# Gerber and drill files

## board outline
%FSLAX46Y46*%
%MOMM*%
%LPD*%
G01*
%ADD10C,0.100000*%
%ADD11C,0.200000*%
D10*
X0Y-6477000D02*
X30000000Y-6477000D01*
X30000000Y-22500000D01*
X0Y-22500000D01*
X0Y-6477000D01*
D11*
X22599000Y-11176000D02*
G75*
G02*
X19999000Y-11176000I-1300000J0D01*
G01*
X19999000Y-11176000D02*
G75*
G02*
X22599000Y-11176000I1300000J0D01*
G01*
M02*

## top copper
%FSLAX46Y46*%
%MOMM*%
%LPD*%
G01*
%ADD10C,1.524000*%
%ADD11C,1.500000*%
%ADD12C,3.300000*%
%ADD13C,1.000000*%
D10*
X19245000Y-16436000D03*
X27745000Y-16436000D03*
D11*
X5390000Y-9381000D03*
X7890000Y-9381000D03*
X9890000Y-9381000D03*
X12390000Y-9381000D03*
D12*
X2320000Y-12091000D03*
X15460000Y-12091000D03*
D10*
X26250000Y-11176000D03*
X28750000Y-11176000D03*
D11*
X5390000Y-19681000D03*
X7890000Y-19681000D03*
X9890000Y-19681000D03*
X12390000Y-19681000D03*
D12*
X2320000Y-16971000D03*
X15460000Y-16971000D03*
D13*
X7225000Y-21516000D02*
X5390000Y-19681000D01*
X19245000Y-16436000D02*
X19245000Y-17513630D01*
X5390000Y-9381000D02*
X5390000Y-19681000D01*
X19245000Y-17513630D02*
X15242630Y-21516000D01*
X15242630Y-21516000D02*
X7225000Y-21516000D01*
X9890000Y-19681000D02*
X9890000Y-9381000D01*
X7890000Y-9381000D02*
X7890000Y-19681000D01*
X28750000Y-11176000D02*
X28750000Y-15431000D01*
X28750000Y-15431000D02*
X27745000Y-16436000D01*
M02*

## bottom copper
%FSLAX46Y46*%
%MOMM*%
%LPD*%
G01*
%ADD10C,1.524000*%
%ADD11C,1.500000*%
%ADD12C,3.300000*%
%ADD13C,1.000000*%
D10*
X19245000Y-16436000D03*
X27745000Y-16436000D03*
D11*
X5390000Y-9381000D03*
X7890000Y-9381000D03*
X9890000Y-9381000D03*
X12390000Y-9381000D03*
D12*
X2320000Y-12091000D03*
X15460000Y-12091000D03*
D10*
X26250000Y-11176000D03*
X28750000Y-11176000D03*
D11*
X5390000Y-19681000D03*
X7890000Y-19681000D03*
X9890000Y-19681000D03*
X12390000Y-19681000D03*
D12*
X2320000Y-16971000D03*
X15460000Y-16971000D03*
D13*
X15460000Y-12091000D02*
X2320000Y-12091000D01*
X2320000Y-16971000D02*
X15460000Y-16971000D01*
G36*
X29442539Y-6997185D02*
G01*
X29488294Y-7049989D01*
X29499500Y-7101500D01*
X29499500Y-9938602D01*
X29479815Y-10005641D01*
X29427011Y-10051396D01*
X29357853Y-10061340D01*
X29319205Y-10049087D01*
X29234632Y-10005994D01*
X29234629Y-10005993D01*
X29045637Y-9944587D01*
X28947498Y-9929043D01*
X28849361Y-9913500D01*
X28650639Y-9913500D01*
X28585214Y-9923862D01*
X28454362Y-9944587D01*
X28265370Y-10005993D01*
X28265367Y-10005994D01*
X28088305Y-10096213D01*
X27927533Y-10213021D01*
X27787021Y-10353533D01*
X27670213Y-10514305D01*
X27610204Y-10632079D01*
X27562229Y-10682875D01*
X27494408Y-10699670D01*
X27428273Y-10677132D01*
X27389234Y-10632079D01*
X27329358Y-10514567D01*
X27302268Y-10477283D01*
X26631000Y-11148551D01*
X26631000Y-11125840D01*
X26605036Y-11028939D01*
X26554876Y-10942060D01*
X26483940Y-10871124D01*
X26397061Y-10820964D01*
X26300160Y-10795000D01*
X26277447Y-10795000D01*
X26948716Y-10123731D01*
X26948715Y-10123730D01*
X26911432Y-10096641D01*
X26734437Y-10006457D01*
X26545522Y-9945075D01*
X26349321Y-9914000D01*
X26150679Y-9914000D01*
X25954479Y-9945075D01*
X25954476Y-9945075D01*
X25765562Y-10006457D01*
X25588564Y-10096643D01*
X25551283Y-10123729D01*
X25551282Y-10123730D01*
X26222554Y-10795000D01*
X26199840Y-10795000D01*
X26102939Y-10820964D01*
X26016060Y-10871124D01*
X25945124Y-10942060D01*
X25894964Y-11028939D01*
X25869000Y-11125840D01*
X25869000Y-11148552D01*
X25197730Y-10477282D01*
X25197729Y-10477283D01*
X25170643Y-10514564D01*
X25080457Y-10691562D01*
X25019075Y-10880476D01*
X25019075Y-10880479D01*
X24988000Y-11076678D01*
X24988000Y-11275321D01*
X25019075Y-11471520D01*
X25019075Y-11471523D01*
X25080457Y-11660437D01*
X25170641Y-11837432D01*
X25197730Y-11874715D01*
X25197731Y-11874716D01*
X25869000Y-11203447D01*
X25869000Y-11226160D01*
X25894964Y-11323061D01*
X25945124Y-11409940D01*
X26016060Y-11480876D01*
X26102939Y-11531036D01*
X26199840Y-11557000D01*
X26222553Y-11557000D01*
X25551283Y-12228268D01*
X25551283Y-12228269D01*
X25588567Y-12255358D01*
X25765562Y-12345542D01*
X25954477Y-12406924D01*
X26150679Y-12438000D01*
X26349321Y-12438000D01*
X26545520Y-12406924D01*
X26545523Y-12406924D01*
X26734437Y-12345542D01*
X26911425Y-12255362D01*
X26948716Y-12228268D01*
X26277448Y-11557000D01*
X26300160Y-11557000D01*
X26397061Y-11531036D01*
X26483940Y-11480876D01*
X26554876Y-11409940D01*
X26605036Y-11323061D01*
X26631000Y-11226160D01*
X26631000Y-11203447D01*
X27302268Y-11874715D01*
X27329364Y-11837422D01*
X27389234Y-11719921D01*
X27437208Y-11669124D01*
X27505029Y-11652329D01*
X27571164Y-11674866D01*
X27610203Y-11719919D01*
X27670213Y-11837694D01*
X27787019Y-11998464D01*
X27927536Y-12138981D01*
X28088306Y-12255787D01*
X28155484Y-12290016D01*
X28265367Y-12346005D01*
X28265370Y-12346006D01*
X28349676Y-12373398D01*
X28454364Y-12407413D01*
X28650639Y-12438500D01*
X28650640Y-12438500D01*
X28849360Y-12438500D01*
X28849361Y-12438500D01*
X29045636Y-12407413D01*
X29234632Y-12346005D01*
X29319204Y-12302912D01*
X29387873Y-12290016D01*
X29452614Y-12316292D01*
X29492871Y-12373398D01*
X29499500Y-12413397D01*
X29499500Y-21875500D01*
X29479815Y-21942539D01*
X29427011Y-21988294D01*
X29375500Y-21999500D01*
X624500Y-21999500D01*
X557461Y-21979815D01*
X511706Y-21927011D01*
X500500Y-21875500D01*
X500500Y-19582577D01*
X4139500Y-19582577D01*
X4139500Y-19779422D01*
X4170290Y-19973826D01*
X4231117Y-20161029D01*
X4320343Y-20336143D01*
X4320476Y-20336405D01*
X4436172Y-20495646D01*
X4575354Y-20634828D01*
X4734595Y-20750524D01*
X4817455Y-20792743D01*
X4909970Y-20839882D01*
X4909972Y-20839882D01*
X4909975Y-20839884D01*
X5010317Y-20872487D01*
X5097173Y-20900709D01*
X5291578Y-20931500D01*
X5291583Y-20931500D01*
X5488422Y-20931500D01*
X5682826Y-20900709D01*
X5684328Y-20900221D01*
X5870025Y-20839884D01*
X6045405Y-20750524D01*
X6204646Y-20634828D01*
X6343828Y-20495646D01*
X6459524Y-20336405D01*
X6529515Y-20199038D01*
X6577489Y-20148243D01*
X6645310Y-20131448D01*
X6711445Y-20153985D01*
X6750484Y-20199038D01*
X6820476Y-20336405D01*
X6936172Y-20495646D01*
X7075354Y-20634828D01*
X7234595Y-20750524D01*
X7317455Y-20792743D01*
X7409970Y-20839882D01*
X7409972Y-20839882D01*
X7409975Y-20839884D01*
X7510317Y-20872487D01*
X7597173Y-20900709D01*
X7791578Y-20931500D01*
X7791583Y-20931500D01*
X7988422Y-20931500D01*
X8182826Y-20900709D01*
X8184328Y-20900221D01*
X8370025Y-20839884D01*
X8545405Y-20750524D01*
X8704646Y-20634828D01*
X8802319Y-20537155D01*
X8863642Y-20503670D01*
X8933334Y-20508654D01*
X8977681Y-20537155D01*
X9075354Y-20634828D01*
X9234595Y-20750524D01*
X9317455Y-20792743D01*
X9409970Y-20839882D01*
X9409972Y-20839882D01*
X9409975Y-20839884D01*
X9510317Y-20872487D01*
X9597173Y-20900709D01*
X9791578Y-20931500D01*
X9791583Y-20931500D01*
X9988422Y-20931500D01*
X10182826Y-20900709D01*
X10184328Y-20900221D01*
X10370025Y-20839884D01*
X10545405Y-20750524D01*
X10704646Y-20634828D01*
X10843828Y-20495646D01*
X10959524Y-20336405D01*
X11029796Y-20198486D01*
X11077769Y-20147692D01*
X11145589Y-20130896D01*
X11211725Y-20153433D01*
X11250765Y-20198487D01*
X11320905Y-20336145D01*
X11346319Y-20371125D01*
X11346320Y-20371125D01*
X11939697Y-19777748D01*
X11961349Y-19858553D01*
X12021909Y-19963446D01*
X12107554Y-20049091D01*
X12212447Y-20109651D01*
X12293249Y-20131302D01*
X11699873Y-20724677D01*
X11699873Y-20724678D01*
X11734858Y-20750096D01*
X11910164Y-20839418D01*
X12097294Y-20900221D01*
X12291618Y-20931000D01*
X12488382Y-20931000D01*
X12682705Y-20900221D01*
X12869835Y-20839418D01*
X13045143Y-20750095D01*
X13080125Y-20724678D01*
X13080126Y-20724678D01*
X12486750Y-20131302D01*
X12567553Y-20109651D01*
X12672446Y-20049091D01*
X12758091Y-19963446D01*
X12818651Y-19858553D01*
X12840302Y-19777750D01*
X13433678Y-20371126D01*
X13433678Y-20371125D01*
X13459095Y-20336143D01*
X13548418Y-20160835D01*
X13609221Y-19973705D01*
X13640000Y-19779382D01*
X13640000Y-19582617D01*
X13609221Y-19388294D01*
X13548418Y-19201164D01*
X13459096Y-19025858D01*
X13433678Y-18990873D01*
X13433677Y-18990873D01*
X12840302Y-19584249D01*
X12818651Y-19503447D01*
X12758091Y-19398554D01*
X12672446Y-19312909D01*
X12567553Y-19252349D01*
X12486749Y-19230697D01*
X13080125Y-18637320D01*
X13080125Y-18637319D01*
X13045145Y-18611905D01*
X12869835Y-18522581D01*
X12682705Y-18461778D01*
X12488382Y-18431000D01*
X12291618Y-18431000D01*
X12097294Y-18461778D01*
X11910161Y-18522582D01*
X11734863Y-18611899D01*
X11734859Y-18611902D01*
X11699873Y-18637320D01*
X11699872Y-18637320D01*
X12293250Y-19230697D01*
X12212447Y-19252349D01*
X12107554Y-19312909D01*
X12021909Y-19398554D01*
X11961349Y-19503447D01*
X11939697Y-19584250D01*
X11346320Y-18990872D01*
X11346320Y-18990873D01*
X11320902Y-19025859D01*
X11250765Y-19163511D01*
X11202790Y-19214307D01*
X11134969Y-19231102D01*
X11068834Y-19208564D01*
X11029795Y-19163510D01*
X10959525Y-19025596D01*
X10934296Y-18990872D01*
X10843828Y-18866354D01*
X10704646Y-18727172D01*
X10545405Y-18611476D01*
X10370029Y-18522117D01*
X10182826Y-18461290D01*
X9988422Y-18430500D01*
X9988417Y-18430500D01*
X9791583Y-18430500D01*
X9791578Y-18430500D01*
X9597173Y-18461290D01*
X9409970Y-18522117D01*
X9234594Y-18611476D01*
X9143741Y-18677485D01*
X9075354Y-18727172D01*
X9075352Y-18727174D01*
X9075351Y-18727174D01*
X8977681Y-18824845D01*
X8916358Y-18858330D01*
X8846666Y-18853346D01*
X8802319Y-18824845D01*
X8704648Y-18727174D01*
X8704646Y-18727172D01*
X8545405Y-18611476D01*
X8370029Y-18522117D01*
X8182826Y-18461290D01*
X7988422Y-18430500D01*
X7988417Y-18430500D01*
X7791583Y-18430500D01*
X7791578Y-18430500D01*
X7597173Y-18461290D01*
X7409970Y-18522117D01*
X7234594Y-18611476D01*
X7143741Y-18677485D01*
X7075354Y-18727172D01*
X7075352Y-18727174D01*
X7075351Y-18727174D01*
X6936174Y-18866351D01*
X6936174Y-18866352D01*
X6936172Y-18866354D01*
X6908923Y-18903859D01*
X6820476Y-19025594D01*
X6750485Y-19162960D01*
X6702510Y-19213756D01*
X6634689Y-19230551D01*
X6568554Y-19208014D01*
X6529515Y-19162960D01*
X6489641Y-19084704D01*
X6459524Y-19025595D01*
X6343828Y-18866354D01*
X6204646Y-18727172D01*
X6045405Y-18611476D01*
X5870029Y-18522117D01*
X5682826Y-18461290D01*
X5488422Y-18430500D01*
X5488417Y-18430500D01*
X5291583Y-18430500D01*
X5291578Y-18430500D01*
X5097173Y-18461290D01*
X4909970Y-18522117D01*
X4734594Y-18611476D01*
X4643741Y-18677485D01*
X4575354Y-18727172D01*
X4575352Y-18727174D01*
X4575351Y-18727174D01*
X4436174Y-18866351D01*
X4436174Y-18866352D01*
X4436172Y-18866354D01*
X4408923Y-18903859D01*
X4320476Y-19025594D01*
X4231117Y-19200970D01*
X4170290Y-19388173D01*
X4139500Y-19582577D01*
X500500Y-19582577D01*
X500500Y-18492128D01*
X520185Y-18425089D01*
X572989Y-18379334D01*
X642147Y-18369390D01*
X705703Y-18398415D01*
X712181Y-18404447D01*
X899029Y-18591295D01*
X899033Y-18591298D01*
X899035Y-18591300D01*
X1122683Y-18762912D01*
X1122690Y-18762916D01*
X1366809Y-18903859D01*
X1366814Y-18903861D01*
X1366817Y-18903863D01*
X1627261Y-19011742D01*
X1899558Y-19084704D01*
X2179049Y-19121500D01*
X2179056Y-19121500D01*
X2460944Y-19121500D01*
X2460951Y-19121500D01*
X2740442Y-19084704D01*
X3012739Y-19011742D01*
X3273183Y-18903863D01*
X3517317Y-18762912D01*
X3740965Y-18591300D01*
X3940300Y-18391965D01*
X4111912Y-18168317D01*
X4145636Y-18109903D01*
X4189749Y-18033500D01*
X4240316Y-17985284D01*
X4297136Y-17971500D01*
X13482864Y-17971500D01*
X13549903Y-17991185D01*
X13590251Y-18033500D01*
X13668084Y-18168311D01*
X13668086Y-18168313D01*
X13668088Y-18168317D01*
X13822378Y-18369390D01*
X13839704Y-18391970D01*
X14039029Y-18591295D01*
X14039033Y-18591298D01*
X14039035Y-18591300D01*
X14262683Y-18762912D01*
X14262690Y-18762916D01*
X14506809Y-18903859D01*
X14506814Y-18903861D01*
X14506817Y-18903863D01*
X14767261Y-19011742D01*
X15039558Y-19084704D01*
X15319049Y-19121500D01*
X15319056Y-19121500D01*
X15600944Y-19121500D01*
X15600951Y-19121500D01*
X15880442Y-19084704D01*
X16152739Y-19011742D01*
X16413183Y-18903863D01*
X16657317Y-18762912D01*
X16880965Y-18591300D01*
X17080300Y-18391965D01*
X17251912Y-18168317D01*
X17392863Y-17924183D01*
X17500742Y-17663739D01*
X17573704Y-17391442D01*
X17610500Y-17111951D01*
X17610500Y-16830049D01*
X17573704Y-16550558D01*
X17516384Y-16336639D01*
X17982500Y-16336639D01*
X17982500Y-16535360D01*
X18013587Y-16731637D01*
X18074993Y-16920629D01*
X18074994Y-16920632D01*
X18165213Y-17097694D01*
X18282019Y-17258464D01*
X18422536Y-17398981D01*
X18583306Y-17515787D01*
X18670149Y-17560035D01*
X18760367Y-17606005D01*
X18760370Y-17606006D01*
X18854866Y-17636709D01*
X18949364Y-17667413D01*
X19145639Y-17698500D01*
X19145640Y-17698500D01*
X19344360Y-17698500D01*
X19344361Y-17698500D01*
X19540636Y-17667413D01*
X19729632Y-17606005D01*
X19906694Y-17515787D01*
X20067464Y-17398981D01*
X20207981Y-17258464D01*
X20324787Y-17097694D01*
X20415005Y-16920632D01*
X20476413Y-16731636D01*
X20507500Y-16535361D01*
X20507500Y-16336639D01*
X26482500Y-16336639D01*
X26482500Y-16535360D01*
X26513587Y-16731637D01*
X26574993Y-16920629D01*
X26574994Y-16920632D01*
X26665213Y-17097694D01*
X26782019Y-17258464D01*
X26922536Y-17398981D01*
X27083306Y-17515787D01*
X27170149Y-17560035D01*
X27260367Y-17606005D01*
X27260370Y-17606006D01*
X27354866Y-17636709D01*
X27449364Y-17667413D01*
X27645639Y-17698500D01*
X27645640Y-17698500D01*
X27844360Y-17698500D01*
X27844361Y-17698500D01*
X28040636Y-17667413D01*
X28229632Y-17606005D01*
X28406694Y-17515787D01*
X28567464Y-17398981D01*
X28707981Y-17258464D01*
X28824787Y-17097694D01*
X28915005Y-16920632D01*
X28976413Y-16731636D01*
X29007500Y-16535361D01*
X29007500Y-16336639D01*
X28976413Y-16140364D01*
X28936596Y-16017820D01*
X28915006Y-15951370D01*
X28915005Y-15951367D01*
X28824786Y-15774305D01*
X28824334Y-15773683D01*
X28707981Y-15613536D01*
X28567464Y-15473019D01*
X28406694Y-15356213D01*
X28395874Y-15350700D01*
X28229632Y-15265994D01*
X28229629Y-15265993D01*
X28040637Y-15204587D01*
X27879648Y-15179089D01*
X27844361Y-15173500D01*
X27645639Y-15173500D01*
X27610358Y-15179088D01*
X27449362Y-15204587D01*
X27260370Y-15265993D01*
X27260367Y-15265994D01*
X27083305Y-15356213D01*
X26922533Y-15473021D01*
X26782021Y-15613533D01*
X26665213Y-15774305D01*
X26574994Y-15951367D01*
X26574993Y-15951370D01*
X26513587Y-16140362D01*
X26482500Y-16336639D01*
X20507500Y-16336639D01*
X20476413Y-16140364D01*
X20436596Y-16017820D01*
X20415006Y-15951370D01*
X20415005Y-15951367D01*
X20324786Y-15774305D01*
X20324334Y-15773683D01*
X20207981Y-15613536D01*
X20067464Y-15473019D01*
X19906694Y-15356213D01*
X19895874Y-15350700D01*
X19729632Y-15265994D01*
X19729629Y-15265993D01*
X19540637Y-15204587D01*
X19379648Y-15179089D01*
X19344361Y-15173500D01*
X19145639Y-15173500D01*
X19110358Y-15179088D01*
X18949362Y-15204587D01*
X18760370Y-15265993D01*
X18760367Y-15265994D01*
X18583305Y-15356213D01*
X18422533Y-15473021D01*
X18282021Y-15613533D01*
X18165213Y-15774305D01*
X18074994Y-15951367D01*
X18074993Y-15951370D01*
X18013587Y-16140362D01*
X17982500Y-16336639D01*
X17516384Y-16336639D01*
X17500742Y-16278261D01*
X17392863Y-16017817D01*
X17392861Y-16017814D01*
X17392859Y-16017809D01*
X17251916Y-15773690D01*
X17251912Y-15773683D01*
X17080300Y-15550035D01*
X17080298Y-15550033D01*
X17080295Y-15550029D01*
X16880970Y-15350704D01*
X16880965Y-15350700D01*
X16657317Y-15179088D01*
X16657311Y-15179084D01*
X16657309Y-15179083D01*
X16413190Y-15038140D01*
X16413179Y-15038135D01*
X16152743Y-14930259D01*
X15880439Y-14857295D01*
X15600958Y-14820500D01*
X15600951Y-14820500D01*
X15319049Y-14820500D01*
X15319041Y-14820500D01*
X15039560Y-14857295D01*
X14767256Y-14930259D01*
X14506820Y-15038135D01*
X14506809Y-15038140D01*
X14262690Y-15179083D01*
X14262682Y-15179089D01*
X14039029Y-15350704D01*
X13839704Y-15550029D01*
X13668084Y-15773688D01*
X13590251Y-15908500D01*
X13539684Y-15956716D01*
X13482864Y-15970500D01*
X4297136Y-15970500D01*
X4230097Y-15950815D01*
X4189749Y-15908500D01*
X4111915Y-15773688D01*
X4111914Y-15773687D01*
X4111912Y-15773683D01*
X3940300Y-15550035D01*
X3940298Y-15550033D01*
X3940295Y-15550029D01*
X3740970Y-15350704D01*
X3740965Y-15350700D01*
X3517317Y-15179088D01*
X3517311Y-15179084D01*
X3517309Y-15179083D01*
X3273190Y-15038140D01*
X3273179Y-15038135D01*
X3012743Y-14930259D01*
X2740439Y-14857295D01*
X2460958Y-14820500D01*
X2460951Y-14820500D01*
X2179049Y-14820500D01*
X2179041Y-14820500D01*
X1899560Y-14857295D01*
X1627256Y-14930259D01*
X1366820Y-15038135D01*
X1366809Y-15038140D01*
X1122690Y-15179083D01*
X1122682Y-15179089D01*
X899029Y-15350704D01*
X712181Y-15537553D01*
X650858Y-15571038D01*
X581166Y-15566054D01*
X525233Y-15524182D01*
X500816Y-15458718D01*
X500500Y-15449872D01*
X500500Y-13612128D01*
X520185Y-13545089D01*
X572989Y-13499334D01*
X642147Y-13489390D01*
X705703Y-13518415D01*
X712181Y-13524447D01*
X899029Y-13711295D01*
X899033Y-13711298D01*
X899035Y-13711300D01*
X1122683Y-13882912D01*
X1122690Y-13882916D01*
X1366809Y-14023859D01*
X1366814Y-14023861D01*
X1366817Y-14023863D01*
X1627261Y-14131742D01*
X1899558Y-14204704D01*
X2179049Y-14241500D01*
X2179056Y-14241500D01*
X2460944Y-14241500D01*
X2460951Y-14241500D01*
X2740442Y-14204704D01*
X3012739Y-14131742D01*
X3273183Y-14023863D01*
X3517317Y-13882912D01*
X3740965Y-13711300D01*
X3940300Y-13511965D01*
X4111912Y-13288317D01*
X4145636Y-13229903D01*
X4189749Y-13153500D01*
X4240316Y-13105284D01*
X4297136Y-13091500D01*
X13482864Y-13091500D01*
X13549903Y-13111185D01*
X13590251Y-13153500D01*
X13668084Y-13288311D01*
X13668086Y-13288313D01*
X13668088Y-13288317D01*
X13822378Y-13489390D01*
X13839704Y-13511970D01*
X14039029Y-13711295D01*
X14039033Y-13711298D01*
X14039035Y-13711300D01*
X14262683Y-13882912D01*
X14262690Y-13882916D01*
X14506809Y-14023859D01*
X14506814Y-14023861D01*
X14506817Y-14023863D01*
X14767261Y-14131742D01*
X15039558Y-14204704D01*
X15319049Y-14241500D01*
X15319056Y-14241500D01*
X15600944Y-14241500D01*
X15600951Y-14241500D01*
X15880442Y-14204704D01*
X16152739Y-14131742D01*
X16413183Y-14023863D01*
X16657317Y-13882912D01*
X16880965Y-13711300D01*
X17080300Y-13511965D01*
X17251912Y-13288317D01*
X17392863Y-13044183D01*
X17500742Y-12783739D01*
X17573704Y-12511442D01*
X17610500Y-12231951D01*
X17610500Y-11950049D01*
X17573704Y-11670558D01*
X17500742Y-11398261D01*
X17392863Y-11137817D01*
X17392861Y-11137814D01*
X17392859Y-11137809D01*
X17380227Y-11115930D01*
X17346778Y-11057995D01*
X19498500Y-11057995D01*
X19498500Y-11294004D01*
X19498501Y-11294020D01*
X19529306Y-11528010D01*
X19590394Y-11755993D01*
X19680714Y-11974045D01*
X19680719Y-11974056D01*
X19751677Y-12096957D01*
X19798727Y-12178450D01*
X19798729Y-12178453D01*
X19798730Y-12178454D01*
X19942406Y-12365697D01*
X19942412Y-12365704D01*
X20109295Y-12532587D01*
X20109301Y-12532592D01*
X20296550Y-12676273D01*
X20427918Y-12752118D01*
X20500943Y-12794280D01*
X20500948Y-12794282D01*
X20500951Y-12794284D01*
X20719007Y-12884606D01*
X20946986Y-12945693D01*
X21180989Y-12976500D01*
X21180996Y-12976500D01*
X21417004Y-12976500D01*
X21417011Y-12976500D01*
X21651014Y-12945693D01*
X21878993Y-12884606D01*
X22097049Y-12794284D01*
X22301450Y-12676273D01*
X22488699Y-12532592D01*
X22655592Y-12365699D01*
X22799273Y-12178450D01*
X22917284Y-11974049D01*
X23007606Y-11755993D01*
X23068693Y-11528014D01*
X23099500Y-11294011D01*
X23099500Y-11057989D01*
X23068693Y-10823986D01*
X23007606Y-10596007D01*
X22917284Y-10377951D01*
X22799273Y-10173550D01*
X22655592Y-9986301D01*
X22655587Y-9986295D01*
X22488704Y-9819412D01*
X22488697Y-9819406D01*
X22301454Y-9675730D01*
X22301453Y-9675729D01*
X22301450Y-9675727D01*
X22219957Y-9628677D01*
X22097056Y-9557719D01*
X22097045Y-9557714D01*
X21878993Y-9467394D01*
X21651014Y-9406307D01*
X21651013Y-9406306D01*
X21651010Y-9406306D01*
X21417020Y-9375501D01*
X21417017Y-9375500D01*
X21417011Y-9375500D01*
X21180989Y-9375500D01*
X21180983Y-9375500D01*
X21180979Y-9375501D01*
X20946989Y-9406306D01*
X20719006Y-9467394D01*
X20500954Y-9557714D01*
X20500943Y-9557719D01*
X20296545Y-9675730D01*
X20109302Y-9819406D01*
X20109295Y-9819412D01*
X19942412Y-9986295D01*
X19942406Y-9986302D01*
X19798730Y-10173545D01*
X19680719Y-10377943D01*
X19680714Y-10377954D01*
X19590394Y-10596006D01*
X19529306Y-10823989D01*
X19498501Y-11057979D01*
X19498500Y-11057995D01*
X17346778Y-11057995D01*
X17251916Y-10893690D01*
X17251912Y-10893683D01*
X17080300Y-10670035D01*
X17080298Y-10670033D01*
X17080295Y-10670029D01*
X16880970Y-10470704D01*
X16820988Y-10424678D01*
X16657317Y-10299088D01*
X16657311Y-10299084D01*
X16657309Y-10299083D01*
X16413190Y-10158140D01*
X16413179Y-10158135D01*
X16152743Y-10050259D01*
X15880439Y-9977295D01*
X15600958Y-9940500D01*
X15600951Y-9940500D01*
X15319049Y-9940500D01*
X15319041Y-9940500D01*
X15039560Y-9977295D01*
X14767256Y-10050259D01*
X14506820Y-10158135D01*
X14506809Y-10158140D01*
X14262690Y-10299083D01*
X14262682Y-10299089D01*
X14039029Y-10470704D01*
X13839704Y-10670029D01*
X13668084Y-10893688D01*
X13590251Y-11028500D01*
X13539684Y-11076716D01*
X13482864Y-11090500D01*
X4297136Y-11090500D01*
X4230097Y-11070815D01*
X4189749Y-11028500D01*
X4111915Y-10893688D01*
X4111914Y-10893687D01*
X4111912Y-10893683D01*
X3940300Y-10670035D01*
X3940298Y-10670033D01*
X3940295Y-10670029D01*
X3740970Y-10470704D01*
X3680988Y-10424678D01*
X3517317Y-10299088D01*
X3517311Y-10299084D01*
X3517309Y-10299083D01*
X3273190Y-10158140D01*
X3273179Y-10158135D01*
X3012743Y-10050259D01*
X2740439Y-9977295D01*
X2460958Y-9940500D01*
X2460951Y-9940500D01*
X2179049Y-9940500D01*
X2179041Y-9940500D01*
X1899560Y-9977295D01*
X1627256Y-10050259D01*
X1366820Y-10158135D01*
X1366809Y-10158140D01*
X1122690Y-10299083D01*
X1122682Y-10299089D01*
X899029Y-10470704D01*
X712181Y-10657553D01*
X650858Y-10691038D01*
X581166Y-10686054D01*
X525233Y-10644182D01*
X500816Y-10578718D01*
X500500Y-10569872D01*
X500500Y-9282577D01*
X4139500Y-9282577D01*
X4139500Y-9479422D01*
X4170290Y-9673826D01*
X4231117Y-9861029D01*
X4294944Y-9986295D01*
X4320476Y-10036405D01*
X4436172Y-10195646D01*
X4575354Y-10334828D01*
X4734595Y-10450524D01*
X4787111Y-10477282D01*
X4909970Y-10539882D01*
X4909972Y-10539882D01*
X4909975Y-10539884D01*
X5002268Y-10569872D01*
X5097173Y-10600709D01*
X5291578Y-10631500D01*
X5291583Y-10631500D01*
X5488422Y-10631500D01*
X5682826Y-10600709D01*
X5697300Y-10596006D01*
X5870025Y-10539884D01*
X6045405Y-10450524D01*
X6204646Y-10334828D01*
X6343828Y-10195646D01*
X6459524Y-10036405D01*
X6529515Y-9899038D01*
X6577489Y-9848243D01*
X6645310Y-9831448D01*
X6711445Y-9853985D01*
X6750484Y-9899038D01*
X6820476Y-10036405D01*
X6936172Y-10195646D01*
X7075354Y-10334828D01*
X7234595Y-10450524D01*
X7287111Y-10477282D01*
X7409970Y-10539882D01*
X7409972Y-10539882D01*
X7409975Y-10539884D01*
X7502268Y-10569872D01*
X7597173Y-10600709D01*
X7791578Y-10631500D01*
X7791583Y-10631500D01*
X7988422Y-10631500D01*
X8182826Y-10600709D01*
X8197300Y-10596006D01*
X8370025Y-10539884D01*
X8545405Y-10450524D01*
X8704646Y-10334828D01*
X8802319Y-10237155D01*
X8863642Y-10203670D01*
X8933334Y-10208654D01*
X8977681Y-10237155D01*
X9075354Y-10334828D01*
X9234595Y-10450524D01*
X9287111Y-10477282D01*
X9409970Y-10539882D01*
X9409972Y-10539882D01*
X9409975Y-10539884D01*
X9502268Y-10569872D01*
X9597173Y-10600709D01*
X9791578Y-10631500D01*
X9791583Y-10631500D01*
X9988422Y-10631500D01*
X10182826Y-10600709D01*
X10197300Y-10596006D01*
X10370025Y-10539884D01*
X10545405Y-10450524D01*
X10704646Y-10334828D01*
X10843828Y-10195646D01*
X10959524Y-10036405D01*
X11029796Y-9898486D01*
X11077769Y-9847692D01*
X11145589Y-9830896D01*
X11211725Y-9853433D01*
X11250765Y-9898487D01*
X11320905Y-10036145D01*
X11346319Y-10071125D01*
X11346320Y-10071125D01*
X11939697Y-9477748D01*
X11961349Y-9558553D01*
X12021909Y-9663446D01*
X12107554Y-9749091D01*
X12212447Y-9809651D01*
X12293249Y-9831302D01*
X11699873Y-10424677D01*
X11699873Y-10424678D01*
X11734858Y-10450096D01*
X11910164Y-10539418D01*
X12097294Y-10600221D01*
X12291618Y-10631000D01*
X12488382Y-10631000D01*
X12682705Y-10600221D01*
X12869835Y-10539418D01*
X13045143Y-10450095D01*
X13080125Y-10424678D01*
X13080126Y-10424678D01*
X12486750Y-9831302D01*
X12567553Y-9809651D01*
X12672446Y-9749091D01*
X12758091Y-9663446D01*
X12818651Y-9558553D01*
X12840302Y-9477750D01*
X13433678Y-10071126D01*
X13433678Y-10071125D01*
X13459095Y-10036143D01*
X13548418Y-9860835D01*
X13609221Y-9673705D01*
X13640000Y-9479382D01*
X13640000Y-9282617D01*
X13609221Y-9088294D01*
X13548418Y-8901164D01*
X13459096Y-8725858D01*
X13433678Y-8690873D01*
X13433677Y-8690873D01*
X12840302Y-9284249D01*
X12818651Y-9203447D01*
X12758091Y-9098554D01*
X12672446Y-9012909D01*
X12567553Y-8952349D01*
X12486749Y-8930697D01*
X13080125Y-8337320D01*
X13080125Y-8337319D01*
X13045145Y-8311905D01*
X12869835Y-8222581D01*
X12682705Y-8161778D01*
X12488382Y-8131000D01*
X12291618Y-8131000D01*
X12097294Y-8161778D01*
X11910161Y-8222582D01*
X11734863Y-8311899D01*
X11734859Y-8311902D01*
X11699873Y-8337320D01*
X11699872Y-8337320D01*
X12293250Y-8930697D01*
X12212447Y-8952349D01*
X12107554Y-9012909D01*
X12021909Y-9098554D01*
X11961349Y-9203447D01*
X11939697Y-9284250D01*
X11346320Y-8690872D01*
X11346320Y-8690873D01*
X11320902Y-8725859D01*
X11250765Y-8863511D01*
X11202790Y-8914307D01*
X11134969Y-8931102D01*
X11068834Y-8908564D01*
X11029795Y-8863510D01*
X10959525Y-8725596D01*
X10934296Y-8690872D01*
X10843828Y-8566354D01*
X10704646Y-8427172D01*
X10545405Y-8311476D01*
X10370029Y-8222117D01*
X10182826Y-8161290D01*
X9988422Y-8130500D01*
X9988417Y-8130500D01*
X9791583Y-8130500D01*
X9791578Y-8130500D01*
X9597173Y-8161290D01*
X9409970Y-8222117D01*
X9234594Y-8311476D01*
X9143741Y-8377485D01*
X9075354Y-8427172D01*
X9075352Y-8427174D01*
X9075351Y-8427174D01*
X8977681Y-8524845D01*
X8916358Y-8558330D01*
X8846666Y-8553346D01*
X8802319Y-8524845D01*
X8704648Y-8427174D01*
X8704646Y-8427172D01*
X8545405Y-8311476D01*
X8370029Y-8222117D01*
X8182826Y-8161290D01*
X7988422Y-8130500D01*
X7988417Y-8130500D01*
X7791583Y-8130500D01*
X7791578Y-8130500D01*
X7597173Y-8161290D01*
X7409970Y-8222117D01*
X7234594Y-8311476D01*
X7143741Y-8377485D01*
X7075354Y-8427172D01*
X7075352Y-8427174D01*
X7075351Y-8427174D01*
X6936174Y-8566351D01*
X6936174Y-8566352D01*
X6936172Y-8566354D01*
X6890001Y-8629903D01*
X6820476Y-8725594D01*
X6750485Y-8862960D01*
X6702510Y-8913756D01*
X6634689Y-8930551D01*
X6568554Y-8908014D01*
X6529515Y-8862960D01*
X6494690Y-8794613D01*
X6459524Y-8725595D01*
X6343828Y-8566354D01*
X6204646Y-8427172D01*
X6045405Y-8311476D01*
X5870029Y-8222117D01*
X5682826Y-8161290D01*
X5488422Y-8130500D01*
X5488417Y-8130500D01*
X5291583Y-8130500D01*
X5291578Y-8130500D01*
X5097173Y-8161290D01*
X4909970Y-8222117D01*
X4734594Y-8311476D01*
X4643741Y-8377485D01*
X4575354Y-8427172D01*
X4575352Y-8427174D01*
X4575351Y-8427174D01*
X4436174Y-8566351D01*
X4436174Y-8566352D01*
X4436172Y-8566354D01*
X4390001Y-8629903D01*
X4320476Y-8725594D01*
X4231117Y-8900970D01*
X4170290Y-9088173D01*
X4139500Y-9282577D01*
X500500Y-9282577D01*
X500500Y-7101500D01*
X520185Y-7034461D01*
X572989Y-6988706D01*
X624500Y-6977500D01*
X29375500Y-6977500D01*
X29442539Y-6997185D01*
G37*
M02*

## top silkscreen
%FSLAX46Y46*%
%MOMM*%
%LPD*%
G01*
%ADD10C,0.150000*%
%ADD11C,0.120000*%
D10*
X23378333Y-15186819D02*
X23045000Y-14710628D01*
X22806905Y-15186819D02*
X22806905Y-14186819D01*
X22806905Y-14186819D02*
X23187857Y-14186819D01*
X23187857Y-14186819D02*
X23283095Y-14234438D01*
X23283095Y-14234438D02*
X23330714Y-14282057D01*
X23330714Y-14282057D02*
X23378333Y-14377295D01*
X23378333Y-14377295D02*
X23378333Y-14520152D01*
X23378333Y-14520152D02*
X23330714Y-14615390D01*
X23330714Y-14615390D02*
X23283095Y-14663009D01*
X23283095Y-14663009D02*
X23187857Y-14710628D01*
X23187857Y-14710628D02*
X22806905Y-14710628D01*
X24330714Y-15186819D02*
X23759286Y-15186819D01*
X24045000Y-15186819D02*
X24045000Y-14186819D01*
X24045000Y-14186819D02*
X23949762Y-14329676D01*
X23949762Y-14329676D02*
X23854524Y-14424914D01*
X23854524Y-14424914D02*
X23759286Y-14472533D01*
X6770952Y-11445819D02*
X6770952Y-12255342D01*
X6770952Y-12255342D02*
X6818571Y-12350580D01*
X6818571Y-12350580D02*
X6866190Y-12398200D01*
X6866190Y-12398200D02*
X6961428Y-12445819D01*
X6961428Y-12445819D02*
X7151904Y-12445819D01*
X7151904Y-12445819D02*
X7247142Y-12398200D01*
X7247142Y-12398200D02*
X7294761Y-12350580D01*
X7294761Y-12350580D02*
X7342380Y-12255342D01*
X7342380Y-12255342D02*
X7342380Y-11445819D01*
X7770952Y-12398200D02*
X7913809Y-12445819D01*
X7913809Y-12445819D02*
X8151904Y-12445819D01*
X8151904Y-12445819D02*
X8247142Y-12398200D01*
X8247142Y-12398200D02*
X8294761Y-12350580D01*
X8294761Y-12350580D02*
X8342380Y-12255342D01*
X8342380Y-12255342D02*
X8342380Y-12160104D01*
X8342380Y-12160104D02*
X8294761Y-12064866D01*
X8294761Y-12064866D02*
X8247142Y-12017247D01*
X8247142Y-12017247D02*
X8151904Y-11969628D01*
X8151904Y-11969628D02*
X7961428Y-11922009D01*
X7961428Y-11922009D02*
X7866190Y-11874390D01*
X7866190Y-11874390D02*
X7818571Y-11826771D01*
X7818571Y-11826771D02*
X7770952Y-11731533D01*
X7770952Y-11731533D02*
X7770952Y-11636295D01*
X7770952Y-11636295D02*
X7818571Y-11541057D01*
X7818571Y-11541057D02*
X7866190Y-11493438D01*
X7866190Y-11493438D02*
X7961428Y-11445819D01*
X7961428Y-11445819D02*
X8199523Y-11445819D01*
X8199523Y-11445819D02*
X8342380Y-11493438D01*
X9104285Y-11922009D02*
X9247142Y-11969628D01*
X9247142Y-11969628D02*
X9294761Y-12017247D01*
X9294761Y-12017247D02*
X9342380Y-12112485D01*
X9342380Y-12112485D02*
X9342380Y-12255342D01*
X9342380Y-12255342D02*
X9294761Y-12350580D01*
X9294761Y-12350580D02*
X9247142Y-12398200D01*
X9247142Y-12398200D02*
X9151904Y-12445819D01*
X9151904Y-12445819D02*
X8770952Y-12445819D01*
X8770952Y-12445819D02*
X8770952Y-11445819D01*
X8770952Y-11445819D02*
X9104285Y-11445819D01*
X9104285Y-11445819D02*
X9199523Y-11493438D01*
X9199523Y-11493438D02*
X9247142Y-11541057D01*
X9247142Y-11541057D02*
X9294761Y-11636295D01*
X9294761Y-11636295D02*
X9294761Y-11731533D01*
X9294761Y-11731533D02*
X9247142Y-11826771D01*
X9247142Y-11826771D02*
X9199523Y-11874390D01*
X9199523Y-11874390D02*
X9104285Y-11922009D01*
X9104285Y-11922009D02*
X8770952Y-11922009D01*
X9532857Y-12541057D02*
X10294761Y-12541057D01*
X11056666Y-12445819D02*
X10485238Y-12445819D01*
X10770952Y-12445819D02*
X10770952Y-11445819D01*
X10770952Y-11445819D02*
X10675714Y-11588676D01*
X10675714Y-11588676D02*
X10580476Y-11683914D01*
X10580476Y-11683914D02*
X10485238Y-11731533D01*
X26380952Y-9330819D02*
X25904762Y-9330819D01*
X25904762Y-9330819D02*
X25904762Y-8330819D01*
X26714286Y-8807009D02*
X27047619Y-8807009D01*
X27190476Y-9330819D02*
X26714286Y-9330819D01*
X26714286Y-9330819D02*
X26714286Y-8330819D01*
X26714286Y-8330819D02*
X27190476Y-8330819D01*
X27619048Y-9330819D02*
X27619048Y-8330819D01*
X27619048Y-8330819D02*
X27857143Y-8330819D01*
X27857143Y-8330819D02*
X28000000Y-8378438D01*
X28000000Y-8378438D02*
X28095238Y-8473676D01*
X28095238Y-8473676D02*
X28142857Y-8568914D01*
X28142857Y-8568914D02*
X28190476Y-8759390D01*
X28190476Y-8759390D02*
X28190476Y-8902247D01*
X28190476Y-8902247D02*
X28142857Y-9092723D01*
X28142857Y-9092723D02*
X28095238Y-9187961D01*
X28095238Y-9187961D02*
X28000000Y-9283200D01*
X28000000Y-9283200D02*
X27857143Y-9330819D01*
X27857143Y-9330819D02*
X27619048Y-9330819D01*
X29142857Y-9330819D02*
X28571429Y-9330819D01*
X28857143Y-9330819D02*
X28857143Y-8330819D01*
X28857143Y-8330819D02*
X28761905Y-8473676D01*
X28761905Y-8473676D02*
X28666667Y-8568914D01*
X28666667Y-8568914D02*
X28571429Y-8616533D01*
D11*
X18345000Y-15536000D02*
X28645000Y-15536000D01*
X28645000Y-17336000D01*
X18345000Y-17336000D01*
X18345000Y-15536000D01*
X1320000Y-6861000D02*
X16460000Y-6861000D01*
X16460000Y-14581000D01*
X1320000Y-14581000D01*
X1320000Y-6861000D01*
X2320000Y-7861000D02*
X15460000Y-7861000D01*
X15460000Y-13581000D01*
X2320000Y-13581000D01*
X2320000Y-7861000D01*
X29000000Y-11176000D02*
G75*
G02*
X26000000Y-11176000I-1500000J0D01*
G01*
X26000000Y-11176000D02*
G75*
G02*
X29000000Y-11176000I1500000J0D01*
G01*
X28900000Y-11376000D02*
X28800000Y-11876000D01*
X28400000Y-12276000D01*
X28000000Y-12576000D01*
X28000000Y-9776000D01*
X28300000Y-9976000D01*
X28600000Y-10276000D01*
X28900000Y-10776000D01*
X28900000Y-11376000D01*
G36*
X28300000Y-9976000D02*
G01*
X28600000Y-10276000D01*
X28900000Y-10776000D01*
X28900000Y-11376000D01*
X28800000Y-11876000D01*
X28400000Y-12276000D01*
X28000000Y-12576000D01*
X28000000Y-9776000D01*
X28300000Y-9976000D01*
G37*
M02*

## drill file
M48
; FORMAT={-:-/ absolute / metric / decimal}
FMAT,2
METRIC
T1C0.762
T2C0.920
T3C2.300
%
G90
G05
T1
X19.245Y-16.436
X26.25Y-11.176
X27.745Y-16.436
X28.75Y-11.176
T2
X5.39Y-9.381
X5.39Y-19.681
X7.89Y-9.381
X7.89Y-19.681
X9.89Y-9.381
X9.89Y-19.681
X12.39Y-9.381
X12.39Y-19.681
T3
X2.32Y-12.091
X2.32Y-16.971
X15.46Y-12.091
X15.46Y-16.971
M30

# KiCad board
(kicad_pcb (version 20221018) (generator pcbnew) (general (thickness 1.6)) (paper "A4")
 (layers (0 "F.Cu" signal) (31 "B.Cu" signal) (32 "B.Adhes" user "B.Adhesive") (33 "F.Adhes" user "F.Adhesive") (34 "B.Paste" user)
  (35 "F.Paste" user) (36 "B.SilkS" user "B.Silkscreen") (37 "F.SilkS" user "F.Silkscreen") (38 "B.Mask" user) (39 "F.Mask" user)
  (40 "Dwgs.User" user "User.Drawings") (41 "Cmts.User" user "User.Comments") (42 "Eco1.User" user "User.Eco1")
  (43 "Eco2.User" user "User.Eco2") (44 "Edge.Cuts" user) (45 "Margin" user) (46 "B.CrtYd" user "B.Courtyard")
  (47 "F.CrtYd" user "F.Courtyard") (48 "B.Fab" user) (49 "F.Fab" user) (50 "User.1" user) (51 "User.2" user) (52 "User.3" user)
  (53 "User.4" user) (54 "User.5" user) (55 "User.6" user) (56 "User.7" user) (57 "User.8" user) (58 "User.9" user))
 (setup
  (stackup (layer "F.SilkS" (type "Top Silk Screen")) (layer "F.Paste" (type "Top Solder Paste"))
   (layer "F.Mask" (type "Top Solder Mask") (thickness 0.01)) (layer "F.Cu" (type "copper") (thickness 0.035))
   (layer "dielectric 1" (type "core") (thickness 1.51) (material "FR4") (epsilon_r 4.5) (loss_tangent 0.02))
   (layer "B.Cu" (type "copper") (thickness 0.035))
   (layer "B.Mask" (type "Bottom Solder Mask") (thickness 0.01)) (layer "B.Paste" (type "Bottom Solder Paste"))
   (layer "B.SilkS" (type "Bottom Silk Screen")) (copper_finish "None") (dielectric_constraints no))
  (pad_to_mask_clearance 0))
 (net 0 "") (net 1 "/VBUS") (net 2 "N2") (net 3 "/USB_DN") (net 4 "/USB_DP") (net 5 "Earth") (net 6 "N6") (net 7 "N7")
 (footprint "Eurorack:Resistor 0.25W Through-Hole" (layer "F.Cu") (at 23.495 16.436)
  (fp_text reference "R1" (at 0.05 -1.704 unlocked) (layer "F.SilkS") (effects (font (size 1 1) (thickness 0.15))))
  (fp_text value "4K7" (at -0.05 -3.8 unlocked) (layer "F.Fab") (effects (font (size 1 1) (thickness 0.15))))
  (fp_rect (start -5.15 -0.9) (end 5.15 0.9) (stroke (width 0.12) (type solid)) (fill none) (layer "F.SilkS"))
  (pad "1" thru_hole circle (at -4.25 0) (size 1.524 1.524) (drill 0.762) (layers "*.Cu" "*.Mask") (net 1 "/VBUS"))
  (pad "2" thru_hole circle (at 4.25 0) (size 1.524 1.524) (drill 0.762) (layers "*.Cu" "*.Mask") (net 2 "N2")))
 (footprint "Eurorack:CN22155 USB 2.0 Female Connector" (layer "F.Cu") (at 2.32 12.091)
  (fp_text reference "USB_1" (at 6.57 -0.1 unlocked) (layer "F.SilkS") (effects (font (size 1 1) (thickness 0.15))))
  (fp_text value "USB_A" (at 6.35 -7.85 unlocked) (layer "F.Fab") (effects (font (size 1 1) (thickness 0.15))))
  (fp_rect (start -1 -5.23) (end 14.14 2.49) (stroke (width 0.12) (type default)) (fill none) (layer "F.SilkS"))
  (fp_rect (start 0 -4.23) (end 13.14 1.49) (stroke (width 0.12) (type default)) (fill none) (layer "F.SilkS"))
  (pad "1" thru_hole circle (at 3.07 -2.71) (size 1.5 1.5) (drill 0.92) (layers "*.Cu" "*.Mask") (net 1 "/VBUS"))
  (pad "2" thru_hole circle (at 5.57 -2.71) (size 1.5 1.5) (drill 0.92) (layers "*.Cu" "*.Mask") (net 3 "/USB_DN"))
  (pad "3" thru_hole circle (at 7.57 -2.71) (size 1.5 1.5) (drill 0.92) (layers "*.Cu" "*.Mask") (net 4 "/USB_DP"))
  (pad "4" thru_hole circle (at 10.07 -2.71) (size 1.5 1.5) (drill 0.92) (layers "*.Cu" "*.Mask") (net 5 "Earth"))
  (pad "5" thru_hole circle (at 0 0) (size 3.3 3.3) (drill 2.3) (layers "*.Cu" "*.Mask") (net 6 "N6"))
  (pad "5" thru_hole circle (at 13.14 0) (size 3.3 3.3) (drill 2.3) (layers "*.Cu" "*.Mask") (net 6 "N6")))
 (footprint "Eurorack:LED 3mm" (layer "F.Cu") (at 27.5 11.176)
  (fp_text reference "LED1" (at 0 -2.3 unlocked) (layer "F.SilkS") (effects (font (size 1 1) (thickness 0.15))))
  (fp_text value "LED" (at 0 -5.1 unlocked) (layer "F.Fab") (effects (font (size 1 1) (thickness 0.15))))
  (fp_circle (center 0 0) (end 0 -1.5) (stroke (width 0.12) (type solid)) (fill none) (layer "F.SilkS"))
  (fp_poly
   (pts (xy 1.4 0.2) (xy 1.3 0.7) (xy 0.9 1.1) (xy 0.5 1.4) (xy 0.5 -1.4) (xy 0.8 -1.2) (xy 1.1 -0.9) (xy 1.4 -0.4))
   (stroke (width 0.12) (type solid)) (fill solid) (layer "F.SilkS"))
  (pad "1" thru_hole circle (at -1.25 0) (size 1.524 1.524) (drill 0.762) (layers "*.Cu" "*.Mask") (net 5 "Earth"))
  (pad "2" thru_hole circle (at 1.25 0) (size 1.524 1.524) (drill 0.762) (layers "*.Cu" "*.Mask") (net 2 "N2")))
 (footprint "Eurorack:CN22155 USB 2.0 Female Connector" (layer "B.Cu") (at 2.32 16.971)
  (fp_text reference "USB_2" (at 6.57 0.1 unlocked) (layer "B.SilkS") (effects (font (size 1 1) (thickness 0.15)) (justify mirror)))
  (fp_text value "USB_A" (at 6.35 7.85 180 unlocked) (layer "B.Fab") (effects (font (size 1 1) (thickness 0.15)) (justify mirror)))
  (pad "1" thru_hole circle (at 3.07 2.71) (size 1.5 1.5) (drill 0.92) (layers "*.Cu" "*.Mask") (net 1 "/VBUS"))
  (pad "2" thru_hole circle (at 5.57 2.71) (size 1.5 1.5) (drill 0.92) (layers "*.Cu" "*.Mask") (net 3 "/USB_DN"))
  (pad "3" thru_hole circle (at 7.57 2.71) (size 1.5 1.5) (drill 0.92) (layers "*.Cu" "*.Mask") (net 4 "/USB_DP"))
  (pad "4" thru_hole circle (at 10.07 2.71) (size 1.5 1.5) (drill 0.92) (layers "*.Cu" "*.Mask") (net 5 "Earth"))
  (pad "5" thru_hole circle (at 0 0) (size 3.3 3.3) (drill 2.3) (layers "*.Cu" "*.Mask") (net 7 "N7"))
  (pad "5" thru_hole circle (at 13.14 0) (size 3.3 3.3) (drill 2.3) (layers "*.Cu" "*.Mask") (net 7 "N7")))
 (gr_rect (start 0 6.477) (end 30 22.5) (stroke (width 0.1) (type default)) (fill none) (layer "Edge.Cuts"))
 (gr_circle (center 21.299 11.176) (end 22.599 11.176) (stroke (width 0.2) (type default)) (fill none) (layer "Edge.Cuts"))
 (segment (start 7.225 21.516) (end 5.39 19.681) (width 1) (layer "F.Cu") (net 1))
 (segment (start 19.245 16.436) (end 19.245 17.51363) (width 1) (layer "F.Cu") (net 1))
 (segment (start 5.39 9.381) (end 5.39 19.681) (width 1) (layer "F.Cu") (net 1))
 (segment (start 19.245 17.51363) (end 15.24263 21.516) (width 1) (layer "F.Cu") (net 1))
 (segment (start 15.24263 21.516) (end 7.225 21.516) (width 1) (layer "F.Cu") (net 1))
 (segment (start 9.89 19.681) (end 9.89 9.381) (width 1) (layer "F.Cu") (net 4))
 (segment (start 7.89 9.381) (end 7.89 19.681) (width 1) (layer "F.Cu") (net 3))
 (segment (start 15.46 12.091) (end 2.32 12.091) (width 1) (layer "B.Cu") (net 6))
 (segment (start 2.32 16.971) (end 15.46 16.971) (width 1) (layer "B.Cu") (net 7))
 (segment (start 28.75 11.176) (end 28.75 15.431) (width 1) (layer "F.Cu") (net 2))
 (segment (start 28.75 15.431) (end 27.745 16.436) (width 1) (layer "F.Cu") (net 2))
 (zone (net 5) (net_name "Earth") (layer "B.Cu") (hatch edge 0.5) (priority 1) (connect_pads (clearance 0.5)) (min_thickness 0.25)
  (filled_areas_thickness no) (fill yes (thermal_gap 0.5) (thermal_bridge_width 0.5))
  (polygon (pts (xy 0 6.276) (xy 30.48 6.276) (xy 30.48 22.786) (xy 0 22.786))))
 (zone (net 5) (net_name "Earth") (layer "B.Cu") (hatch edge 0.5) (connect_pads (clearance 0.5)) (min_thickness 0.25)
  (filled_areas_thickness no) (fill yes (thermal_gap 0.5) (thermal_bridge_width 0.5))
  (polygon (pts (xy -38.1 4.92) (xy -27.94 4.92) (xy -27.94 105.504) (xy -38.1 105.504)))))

